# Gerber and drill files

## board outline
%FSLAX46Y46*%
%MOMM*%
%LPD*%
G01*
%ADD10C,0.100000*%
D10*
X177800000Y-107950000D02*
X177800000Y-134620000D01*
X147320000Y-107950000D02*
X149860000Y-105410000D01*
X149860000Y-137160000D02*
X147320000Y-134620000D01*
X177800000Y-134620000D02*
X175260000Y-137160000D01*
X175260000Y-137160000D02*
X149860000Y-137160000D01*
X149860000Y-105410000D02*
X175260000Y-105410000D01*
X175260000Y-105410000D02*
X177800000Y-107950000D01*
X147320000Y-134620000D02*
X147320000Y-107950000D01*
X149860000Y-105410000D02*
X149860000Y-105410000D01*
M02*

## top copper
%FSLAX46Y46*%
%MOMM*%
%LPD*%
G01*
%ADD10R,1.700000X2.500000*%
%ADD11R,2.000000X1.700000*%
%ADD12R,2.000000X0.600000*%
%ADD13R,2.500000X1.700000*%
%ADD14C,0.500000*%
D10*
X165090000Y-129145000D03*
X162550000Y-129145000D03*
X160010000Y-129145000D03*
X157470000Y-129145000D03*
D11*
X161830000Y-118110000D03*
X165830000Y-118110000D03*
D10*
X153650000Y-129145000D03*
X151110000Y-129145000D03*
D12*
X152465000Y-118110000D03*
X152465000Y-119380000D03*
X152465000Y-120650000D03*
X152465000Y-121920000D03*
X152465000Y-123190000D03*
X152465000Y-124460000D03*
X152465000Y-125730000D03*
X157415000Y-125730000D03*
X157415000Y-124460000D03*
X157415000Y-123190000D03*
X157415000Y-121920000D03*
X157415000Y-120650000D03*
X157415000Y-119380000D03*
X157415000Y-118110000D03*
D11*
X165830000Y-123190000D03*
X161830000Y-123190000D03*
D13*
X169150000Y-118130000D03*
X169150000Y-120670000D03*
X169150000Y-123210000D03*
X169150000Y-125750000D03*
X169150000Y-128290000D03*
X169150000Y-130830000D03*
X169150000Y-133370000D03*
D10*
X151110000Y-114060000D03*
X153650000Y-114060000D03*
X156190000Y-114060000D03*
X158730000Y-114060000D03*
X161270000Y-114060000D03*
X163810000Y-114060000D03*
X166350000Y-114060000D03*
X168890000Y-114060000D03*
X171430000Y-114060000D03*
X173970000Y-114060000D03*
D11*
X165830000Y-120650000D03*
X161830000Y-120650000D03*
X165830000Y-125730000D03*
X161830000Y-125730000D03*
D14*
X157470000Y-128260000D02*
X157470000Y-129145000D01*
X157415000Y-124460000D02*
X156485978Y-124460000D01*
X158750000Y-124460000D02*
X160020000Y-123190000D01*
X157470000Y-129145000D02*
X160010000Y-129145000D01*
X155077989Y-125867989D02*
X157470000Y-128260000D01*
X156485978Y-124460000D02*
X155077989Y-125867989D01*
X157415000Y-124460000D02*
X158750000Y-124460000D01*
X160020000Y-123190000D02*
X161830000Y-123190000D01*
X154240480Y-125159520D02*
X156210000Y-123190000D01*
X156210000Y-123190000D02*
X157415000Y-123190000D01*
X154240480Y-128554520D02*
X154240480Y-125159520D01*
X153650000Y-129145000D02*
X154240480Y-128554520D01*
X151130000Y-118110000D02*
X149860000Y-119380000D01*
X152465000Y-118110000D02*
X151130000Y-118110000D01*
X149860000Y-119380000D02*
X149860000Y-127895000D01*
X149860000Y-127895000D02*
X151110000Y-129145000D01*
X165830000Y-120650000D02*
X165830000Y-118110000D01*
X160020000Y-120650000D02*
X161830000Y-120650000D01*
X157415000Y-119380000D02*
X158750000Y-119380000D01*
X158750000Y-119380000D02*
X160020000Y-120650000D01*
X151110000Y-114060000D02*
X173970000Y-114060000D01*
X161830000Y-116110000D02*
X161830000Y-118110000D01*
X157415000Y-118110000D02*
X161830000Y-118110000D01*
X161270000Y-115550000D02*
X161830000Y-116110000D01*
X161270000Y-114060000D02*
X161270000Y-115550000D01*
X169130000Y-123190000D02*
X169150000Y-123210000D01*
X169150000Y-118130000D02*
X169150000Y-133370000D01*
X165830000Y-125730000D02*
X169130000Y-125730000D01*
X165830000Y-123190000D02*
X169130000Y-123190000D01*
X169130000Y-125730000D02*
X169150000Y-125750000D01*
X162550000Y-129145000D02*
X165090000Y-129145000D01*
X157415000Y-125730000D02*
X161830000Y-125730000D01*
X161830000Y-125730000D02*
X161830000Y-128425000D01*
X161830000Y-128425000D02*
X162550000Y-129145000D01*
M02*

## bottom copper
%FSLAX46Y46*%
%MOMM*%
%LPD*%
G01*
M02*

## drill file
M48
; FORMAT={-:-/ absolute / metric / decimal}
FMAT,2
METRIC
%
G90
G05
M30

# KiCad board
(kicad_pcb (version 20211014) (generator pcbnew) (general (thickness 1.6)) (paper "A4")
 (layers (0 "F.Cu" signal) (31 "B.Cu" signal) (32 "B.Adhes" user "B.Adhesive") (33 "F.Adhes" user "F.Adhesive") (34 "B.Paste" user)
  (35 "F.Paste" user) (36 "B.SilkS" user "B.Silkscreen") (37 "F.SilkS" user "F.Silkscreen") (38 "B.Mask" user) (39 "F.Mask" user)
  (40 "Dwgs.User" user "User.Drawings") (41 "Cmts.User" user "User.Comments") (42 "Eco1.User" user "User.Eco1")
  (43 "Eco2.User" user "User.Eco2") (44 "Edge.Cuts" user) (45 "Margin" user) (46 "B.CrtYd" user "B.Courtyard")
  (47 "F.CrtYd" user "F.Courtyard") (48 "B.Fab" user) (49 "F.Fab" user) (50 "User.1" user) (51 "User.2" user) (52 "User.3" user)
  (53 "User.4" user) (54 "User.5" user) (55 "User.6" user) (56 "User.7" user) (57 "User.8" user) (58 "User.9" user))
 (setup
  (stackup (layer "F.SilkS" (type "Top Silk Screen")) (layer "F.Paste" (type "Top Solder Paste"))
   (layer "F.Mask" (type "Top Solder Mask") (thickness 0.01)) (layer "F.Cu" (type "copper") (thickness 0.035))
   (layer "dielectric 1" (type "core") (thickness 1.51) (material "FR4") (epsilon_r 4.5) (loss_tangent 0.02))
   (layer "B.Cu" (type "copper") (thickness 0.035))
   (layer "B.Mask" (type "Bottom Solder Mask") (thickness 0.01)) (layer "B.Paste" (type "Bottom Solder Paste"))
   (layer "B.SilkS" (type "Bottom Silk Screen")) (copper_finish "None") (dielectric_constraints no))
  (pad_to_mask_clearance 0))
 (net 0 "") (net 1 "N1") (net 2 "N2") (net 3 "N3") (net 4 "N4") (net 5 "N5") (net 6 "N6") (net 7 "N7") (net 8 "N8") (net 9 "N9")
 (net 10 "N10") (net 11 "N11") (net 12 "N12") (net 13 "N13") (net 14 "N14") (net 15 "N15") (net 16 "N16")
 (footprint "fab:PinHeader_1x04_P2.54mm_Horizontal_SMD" (layer "F.Cu") (at 165.09 129.145 -90)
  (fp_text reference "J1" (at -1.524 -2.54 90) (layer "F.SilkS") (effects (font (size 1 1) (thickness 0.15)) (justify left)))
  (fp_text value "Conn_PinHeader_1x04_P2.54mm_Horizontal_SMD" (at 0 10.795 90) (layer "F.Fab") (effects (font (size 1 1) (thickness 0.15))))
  (pad "1" smd rect locked (at 0 0 270) (size 2.5 1.7) (layers "F.Cu" "F.Paste" "F.Mask") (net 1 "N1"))
  (pad "2" smd rect locked (at 0 2.54 270) (size 2.5 1.7) (layers "F.Cu" "F.Paste" "F.Mask") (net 1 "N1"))
  (pad "3" smd rect locked (at 0 5.08 270) (size 2.5 1.7) (layers "F.Cu" "F.Paste" "F.Mask") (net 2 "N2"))
  (pad "4" smd rect locked (at 0 7.62 270) (size 2.5 1.7) (layers "F.Cu" "F.Paste" "F.Mask") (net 2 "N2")))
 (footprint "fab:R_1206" (layer "F.Cu") (at 163.83 118.11)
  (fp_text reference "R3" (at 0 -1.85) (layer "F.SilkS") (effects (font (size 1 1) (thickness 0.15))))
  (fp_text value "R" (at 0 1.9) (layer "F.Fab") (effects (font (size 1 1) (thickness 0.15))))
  (pad "1" smd rect locked (at -2 0) (size 2 1.7) (layers "F.Cu" "F.Paste" "F.Mask") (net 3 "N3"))
  (pad "2" smd rect locked (at 2 0) (size 2 1.7) (layers "F.Cu" "F.Paste" "F.Mask") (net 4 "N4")))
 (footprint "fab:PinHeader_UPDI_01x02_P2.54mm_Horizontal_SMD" (layer "F.Cu") (at 153.65 129.145 -90)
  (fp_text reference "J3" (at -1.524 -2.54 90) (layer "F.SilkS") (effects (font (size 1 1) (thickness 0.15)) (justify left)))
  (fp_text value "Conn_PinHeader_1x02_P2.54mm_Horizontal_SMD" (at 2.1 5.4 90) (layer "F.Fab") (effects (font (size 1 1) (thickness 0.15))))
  (pad "1" smd rect locked (at 0 0 270) (size 2.5 1.7) (layers "F.Cu" "F.Paste" "F.Mask") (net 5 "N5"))
  (pad "2" smd rect locked (at 0 2.54 270) (size 2.5 1.7) (layers "F.Cu" "F.Paste" "F.Mask") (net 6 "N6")))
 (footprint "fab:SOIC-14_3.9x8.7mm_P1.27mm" (layer "F.Cu") (at 154.94 121.92)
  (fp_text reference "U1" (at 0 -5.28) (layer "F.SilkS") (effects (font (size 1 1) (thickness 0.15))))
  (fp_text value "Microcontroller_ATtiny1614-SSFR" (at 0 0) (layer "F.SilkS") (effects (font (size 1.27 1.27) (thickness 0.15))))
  (pad "1" smd rect (at -2.475 -3.81) (size 2 0.6) (layers "F.Cu" "F.Paste" "F.Mask") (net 6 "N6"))
  (pad "2" smd rect (at -2.475 -2.54) (size 2 0.6) (layers "F.Cu" "F.Paste" "F.Mask") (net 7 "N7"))
  (pad "3" smd rect (at -2.475 -1.27) (size 2 0.6) (layers "F.Cu" "F.Paste" "F.Mask") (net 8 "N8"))
  (pad "4" smd rect (at -2.475 0) (size 2 0.6) (layers "F.Cu" "F.Paste" "F.Mask") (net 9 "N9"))
  (pad "5" smd rect (at -2.475 1.27) (size 2 0.6) (layers "F.Cu" "F.Paste" "F.Mask") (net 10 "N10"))
  (pad "6" smd rect (at -2.475 2.54) (size 2 0.6) (layers "F.Cu" "F.Paste" "F.Mask") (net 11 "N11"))
  (pad "7" smd rect (at -2.475 3.81) (size 2 0.6) (layers "F.Cu" "F.Paste" "F.Mask") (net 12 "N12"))
  (pad "8" smd rect (at 2.475 3.81) (size 2 0.6) (layers "F.Cu" "F.Paste" "F.Mask") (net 1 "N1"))
  (pad "9" smd rect (at 2.475 2.54) (size 2 0.6) (layers "F.Cu" "F.Paste" "F.Mask") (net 2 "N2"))
  (pad "10" smd rect (at 2.475 1.27) (size 2 0.6) (layers "F.Cu" "F.Paste" "F.Mask") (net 5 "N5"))
  (pad "11" smd rect (at 2.475 0) (size 2 0.6) (layers "F.Cu" "F.Paste" "F.Mask") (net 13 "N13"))
  (pad "12" smd rect (at 2.475 -1.27) (size 2 0.6) (layers "F.Cu" "F.Paste" "F.Mask") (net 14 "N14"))
  (pad "13" smd rect (at 2.475 -2.54) (size 2 0.6) (layers "F.Cu" "F.Paste" "F.Mask") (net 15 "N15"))
  (pad "14" smd rect (at 2.475 -3.81) (size 2 0.6) (layers "F.Cu" "F.Paste" "F.Mask") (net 3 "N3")))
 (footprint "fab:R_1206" (layer "F.Cu") (at 163.83 123.19 180)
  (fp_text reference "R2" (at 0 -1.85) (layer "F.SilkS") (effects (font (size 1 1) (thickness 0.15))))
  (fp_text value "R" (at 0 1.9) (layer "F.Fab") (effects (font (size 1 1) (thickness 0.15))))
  (pad "1" smd rect locked (at -2 0 180) (size 2 1.7) (layers "F.Cu" "F.Paste" "F.Mask") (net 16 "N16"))
  (pad "2" smd rect locked (at 2 0 180) (size 2 1.7) (layers "F.Cu" "F.Paste" "F.Mask") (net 2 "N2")))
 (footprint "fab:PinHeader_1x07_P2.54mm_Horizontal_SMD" (layer "F.Cu") (at 169.15 118.13)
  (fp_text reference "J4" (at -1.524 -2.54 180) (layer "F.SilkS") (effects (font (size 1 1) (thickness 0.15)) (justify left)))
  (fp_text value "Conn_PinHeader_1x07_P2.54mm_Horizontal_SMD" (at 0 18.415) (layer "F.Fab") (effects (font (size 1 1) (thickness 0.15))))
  (pad "1" smd rect locked (at 0 0) (size 2.5 1.7) (layers "F.Cu" "F.Paste" "F.Mask") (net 16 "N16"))
  (pad "2" smd rect locked (at 0 2.54) (size 2.5 1.7) (layers "F.Cu" "F.Paste" "F.Mask") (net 16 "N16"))
  (pad "3" smd rect locked (at 0 5.08) (size 2.5 1.7) (layers "F.Cu" "F.Paste" "F.Mask") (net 16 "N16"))
  (pad "4" smd rect locked (at 0 7.62) (size 2.5 1.7) (layers "F.Cu" "F.Paste" "F.Mask") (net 16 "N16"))
  (pad "5" smd rect locked (at 0 10.16) (size 2.5 1.7) (layers "F.Cu" "F.Paste" "F.Mask") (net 16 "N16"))
  (pad "6" smd rect locked (at 0 12.7) (size 2.5 1.7) (layers "F.Cu" "F.Paste" "F.Mask") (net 16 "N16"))
  (pad "7" smd rect locked (at 0 15.24) (size 2.5 1.7) (layers "F.Cu" "F.Paste" "F.Mask") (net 16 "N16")))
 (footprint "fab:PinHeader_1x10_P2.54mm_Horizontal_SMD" (layer "F.Cu") (at 151.11 114.06 90)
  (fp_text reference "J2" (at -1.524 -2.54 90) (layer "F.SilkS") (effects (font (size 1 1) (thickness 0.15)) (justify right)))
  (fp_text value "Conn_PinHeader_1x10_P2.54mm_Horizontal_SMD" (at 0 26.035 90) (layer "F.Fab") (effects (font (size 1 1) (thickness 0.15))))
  (pad "1" smd rect locked (at 0 0 90) (size 2.5 1.7) (layers "F.Cu" "F.Paste" "F.Mask") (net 3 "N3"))
  (pad "2" smd rect locked (at 0 2.54 90) (size 2.5 1.7) (layers "F.Cu" "F.Paste" "F.Mask") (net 3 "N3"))
  (pad "3" smd rect locked (at 0 5.08 90) (size 2.5 1.7) (layers "F.Cu" "F.Paste" "F.Mask") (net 3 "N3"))
  (pad "4" smd rect locked (at 0 7.62 90) (size 2.5 1.7) (layers "F.Cu" "F.Paste" "F.Mask") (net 3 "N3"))
  (pad "5" smd rect locked (at 0 10.16 90) (size 2.5 1.7) (layers "F.Cu" "F.Paste" "F.Mask") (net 3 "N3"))
  (pad "6" smd rect locked (at 0 12.7 90) (size 2.5 1.7) (layers "F.Cu" "F.Paste" "F.Mask") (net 3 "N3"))
  (pad "7" smd rect locked (at 0 15.24 90) (size 2.5 1.7) (layers "F.Cu" "F.Paste" "F.Mask") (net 3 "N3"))
  (pad "8" smd rect locked (at 0 17.78 90) (size 2.5 1.7) (layers "F.Cu" "F.Paste" "F.Mask") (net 3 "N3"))
  (pad "9" smd rect locked (at 0 20.32 90) (size 2.5 1.7) (layers "F.Cu" "F.Paste" "F.Mask") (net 3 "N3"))
  (pad "10" smd rect locked (at 0 22.86 90) (size 2.5 1.7) (layers "F.Cu" "F.Paste" "F.Mask") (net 3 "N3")))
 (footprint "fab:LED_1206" (layer "F.Cu") (at 163.83 120.65 180)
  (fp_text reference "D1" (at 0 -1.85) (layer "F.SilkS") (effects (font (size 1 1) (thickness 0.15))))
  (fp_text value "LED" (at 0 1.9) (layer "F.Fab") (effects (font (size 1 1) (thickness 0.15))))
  (pad "1" smd rect locked (at -2 0 180) (size 2 1.7) (layers "F.Cu" "F.Paste" "F.Mask") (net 4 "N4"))
  (pad "2" smd rect locked (at 2 0 180) (size 2 1.7) (layers "F.Cu" "F.Paste" "F.Mask") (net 15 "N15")))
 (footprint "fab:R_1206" (layer "F.Cu") (at 163.83 125.73 180)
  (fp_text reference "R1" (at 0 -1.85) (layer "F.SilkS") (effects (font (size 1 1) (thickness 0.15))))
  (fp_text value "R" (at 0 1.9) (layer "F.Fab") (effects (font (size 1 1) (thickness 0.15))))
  (pad "1" smd rect locked (at -2 0 180) (size 2 1.7) (layers "F.Cu" "F.Paste" "F.Mask") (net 16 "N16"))
  (pad "2" smd rect locked (at 2 0 180) (size 2 1.7) (layers "F.Cu" "F.Paste" "F.Mask") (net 1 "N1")))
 (gr_line (start 177.8 107.95) (end 177.8 134.62) (layer "Edge.Cuts") (width 0.1))
 (gr_line (start 147.32 107.95) (end 149.86 105.41) (layer "Edge.Cuts") (width 0.1))
 (gr_line (start 149.86 137.16) (end 147.32 134.62) (layer "Edge.Cuts") (width 0.1))
 (gr_line (start 177.8 134.62) (end 175.26 137.16) (layer "Edge.Cuts") (width 0.1))
 (gr_line (start 175.26 137.16) (end 149.86 137.16) (layer "Edge.Cuts") (width 0.1))
 (gr_line (start 149.86 105.41) (end 175.26 105.41) (layer "Edge.Cuts") (width 0.1))
 (gr_line (start 175.26 105.41) (end 177.8 107.95) (layer "Edge.Cuts") (width 0.1))
 (gr_line (start 147.32 134.62) (end 147.32 107.95) (layer "Edge.Cuts") (width 0.1))
 (gr_line (start 149.86 105.41) (end 149.86 105.41) (layer "Edge.Cuts") (width 0.1))
 (segment (start 157.47 128.26) (end 157.47 129.145) (width 0.5) (layer "F.Cu") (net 2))
 (segment (start 157.415 124.46) (end 156.485978 124.46) (width 0.5) (layer "F.Cu") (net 2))
 (segment (start 158.75 124.46) (end 160.02 123.19) (width 0.5) (layer "F.Cu") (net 2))
 (segment (start 157.47 129.145) (end 160.01 129.145) (width 0.5) (layer "F.Cu") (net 2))
 (segment (start 155.077989 125.867989) (end 157.47 128.26) (width 0.5) (layer "F.Cu") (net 2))
 (segment (start 156.485978 124.46) (end 155.077989 125.867989) (width 0.5) (layer "F.Cu") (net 2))
 (segment (start 157.415 124.46) (end 158.75 124.46) (width 0.5) (layer "F.Cu") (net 2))
 (segment (start 160.02 123.19) (end 161.83 123.19) (width 0.5) (layer "F.Cu") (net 2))
 (segment (start 154.24048 125.15952) (end 156.21 123.19) (width 0.5) (layer "F.Cu") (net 5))
 (segment (start 156.21 123.19) (end 157.415 123.19) (width 0.5) (layer "F.Cu") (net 5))
 (segment (start 154.24048 128.55452) (end 154.24048 125.15952) (width 0.5) (layer "F.Cu") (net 5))
 (segment (start 153.65 129.145) (end 154.24048 128.55452) (width 0.5) (layer "F.Cu") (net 5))
 (segment (start 151.13 118.11) (end 149.86 119.38) (width 0.5) (layer "F.Cu") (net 6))
 (segment (start 152.465 118.11) (end 151.13 118.11) (width 0.5) (layer "F.Cu") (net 6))
 (segment (start 149.86 119.38) (end 149.86 127.895) (width 0.5) (layer "F.Cu") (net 6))
 (segment (start 149.86 127.895) (end 151.11 129.145) (width 0.5) (layer "F.Cu") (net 6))
 (segment (start 165.83 120.65) (end 165.83 118.11) (width 0.5) (layer "F.Cu") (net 4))
 (segment (start 160.02 120.65) (end 161.83 120.65) (width 0.5) (layer "F.Cu") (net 15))
 (segment (start 157.415 119.38) (end 158.75 119.38) (width 0.5) (layer "F.Cu") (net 15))
 (segment (start 158.75 119.38) (end 160.02 120.65) (width 0.5) (layer "F.Cu") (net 15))
 (segment (start 151.11 114.06) (end 173.97 114.06) (width 0.5) (layer "F.Cu") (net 3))
 (segment (start 161.83 116.11) (end 161.83 118.11) (width 0.5) (layer "F.Cu") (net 3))
 (segment (start 157.415 118.11) (end 161.83 118.11) (width 0.5) (layer "F.Cu") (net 3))
 (segment (start 161.27 115.55) (end 161.83 116.11) (width 0.5) (layer "F.Cu") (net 3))
 (segment (start 161.27 114.06) (end 161.27 115.55) (width 0.5) (layer "F.Cu") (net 3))
 (segment (start 169.13 123.19) (end 169.15 123.21) (width 0.5) (layer "F.Cu") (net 16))
 (segment (start 169.15 118.13) (end 169.15 133.37) (width 0.5) (layer "F.Cu") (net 16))
 (segment (start 165.83 125.73) (end 169.13 125.73) (width 0.5) (layer "F.Cu") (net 16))
 (segment (start 165.83 123.19) (end 169.13 123.19) (width 0.5) (layer "F.Cu") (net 16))
 (segment (start 169.13 125.73) (end 169.15 125.75) (width 0.5) (layer "F.Cu") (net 16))
 (segment (start 162.55 129.145) (end 165.09 129.145) (width 0.5) (layer "F.Cu") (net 1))
 (segment (start 157.415 125.73) (end 161.83 125.73) (width 0.5) (layer "F.Cu") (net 1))
 (segment (start 161.83 125.73) (end 161.83 128.425) (width 0.5) (layer "F.Cu") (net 1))
 (segment (start 161.83 128.425) (end 162.55 129.145) (width 0.5) (layer "F.Cu") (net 1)))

